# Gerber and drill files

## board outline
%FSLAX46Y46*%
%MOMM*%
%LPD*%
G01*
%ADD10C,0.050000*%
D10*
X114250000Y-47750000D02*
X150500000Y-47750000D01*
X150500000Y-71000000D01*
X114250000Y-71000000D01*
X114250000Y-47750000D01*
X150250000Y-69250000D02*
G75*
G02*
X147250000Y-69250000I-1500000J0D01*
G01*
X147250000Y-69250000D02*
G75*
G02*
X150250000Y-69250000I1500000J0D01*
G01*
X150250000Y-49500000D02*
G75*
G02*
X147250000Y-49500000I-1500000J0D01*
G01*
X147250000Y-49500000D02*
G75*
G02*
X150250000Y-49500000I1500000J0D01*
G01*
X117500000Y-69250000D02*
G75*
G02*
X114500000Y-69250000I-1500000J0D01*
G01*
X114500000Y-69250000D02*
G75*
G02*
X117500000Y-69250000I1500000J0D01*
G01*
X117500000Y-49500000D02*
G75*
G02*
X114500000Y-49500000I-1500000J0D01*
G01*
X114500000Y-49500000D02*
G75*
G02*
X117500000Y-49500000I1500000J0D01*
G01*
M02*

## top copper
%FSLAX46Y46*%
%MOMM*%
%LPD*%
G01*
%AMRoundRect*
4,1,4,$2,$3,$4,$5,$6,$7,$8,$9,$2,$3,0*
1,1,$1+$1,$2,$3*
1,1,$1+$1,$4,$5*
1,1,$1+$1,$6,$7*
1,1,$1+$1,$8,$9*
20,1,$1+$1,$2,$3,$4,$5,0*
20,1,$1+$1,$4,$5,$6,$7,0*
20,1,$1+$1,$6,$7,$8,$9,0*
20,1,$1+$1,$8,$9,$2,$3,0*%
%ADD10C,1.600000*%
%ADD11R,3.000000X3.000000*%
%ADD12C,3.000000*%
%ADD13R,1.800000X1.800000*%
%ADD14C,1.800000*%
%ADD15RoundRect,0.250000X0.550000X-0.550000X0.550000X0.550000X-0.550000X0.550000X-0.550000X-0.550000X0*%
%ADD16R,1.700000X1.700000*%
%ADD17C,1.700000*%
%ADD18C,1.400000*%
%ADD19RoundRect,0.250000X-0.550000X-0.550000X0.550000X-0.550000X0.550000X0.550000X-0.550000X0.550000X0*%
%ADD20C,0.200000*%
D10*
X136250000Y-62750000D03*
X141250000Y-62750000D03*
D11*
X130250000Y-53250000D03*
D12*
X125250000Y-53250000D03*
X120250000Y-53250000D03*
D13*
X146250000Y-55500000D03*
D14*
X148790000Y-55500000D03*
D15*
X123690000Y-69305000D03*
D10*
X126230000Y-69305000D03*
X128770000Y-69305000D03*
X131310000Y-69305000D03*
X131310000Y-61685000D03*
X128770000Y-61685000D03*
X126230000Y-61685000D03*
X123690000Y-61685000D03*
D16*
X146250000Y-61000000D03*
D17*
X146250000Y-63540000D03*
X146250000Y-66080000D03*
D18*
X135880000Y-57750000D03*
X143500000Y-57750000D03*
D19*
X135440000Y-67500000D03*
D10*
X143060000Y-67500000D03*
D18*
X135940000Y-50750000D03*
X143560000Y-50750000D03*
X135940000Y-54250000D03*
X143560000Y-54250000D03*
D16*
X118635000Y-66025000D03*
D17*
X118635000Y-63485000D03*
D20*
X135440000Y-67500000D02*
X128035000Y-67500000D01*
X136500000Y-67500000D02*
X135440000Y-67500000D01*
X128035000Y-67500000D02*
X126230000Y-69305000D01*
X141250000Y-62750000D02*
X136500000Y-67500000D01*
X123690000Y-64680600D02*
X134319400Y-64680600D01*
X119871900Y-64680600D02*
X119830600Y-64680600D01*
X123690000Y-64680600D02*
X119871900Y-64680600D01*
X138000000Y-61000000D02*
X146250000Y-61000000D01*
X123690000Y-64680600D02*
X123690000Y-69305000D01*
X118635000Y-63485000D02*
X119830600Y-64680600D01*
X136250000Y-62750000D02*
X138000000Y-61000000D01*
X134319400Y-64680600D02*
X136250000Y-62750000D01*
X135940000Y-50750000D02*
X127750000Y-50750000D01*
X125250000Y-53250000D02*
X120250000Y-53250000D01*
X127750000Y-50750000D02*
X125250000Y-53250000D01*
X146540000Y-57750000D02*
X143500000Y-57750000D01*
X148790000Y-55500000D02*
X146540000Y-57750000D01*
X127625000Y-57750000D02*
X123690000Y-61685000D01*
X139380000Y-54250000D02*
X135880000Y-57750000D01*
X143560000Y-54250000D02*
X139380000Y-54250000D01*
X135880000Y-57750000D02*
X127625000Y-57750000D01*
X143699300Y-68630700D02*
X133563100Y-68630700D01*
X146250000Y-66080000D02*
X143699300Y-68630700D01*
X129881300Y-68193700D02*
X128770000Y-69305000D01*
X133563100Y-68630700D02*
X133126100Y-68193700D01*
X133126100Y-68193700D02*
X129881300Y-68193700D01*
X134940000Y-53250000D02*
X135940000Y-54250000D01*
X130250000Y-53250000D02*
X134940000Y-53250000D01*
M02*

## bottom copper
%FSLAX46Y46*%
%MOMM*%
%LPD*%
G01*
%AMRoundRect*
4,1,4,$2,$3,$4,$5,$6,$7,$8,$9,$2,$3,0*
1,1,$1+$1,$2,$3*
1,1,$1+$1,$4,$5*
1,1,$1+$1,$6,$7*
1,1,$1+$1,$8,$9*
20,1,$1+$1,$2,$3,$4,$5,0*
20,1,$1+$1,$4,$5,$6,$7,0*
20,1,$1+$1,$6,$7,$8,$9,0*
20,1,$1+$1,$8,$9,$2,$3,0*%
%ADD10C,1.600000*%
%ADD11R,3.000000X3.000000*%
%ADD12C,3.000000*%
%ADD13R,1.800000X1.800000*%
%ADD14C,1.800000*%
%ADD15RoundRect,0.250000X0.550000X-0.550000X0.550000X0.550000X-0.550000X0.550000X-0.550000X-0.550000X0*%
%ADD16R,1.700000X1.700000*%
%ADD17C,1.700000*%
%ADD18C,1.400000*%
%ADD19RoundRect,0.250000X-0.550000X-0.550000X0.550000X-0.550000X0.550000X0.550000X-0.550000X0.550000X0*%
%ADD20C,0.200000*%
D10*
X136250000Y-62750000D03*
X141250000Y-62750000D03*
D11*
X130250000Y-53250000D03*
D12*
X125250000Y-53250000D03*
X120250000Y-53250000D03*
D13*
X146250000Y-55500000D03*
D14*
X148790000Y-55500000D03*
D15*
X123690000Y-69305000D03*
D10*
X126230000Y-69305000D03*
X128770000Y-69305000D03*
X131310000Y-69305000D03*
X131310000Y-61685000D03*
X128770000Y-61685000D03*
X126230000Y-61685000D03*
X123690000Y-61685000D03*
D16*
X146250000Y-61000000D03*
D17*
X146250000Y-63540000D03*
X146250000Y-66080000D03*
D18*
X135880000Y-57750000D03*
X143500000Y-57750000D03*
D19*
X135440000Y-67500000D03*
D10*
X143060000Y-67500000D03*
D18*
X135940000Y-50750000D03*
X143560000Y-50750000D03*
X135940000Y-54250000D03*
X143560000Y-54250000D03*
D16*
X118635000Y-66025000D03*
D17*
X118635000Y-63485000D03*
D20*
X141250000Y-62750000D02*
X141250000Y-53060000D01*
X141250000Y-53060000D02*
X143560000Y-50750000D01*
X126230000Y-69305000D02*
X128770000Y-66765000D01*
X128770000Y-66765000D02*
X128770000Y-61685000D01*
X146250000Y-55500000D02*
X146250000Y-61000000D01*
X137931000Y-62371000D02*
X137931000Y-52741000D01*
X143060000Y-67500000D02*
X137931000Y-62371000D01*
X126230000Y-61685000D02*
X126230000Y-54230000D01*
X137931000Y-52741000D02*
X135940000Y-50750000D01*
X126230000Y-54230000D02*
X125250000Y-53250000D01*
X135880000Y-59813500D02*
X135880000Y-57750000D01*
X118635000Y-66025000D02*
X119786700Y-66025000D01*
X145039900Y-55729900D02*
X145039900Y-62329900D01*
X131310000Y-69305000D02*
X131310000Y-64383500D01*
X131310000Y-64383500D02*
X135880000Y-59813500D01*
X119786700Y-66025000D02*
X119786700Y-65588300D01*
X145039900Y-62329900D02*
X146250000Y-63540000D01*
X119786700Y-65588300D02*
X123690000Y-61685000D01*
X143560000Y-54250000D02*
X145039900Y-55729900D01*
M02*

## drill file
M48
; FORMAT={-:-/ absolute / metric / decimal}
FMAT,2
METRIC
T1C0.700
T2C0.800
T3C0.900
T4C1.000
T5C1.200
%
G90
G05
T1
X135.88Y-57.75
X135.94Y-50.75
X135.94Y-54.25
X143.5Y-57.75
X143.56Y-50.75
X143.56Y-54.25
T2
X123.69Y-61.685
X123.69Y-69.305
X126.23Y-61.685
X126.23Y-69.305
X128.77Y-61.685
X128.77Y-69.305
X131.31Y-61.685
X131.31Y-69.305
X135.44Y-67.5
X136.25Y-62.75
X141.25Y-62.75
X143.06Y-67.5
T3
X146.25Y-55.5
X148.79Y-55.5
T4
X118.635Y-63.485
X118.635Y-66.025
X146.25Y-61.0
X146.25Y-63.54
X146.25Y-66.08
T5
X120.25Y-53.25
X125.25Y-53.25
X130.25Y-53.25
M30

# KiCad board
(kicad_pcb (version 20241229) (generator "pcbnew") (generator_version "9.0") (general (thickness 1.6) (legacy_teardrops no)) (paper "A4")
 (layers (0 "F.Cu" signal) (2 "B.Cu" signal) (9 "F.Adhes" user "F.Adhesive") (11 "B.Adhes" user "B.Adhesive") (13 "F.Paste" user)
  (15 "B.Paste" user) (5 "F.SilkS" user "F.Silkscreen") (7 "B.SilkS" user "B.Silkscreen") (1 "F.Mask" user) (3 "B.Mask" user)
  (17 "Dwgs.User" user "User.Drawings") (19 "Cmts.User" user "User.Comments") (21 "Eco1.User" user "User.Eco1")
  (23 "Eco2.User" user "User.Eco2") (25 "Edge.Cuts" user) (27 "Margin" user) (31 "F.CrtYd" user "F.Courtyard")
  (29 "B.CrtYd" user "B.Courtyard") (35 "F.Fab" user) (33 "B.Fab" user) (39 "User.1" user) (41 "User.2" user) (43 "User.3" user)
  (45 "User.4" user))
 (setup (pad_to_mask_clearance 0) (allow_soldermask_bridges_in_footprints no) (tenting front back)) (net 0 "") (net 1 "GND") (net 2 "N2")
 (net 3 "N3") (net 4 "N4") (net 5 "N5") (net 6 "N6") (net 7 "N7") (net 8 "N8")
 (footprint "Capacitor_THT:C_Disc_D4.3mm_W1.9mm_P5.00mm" (layer "F.Cu") (at 136.25 62.75)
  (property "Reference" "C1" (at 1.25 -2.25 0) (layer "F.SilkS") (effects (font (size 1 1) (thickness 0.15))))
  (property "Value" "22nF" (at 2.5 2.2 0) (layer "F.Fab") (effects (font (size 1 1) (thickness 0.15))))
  (pad "1" thru_hole circle (at 0 0) (size 1.6 1.6) (drill 0.8) (layers "*.Cu" "*.Mask") (remove_unused_layers no) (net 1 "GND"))
  (pad "2" thru_hole circle (at 5 0) (size 1.6 1.6) (drill 0.8) (layers "*.Cu" "*.Mask") (remove_unused_layers no) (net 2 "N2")))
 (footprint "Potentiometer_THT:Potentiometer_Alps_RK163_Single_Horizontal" (layer "F.Cu") (at 130.25 53.25 -90)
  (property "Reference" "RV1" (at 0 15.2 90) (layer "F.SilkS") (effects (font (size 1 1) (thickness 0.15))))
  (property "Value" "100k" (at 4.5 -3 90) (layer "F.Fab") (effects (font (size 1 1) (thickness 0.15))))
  (pad "1" thru_hole rect (at 0 0 90) (size 3 3) (drill 1.2) (layers "*.Cu" "*.Mask") (remove_unused_layers no) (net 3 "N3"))
  (pad "2" thru_hole circle (at 0 5 90) (size 3 3) (drill 1.2) (layers "*.Cu" "*.Mask") (remove_unused_layers no) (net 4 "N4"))
  (pad "3" thru_hole circle (at 0 10 90) (size 3 3) (drill 1.2) (layers "*.Cu" "*.Mask") (remove_unused_layers no) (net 4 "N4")))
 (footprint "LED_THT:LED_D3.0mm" (layer "F.Cu") (at 146.25 55.5)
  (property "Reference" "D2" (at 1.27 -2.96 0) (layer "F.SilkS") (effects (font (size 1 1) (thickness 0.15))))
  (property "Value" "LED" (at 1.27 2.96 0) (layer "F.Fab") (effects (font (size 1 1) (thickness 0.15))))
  (pad "1" thru_hole rect (at 0 0) (size 1.8 1.8) (drill 0.9) (layers "*.Cu" "*.Mask") (remove_unused_layers no) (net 1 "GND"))
  (pad "2" thru_hole circle (at 2.54 0) (size 1.8 1.8) (drill 0.9) (layers "*.Cu" "*.Mask") (remove_unused_layers no) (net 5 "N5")))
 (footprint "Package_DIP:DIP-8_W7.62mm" (layer "F.Cu") (at 123.69 69.305 90)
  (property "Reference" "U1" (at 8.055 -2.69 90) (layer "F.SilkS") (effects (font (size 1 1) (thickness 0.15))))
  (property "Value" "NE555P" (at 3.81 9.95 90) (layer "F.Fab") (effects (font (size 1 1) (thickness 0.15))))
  (pad "1" thru_hole roundrect (at 0 0 90) (size 1.6 1.6) (drill 0.8) (layers "*.Cu" "*.Mask") (remove_unused_layers no)
   (roundrect_rratio 0.15625) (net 1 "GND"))
  (pad "2" thru_hole circle (at 0 2.54 90) (size 1.6 1.6) (drill 0.8) (layers "*.Cu" "*.Mask") (remove_unused_layers no) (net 2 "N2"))
  (pad "3" thru_hole circle (at 0 5.08 90) (size 1.6 1.6) (drill 0.8) (layers "*.Cu" "*.Mask") (remove_unused_layers no) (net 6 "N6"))
  (pad "4" thru_hole circle (at 0 7.62 90) (size 1.6 1.6) (drill 0.8) (layers "*.Cu" "*.Mask") (remove_unused_layers no) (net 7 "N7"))
  (pad "5" thru_hole circle (at 7.62 7.62 90) (size 1.6 1.6) (drill 0.8) (layers "*.Cu" "*.Mask") (remove_unused_layers no) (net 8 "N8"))
  (pad "6" thru_hole circle (at 7.62 5.08 90) (size 1.6 1.6) (drill 0.8) (layers "*.Cu" "*.Mask") (remove_unused_layers no) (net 2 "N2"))
  (pad "7" thru_hole circle (at 7.62 2.54 90) (size 1.6 1.6) (drill 0.8) (layers "*.Cu" "*.Mask") (remove_unused_layers no) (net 4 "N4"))
  (pad "8" thru_hole circle (at 7.62 0 90) (size 1.6 1.6) (drill 0.8) (layers "*.Cu" "*.Mask") (remove_unused_layers no) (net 7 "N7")))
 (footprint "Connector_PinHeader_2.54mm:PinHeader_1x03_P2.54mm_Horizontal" (layer "F.Cu") (at 146.25 61)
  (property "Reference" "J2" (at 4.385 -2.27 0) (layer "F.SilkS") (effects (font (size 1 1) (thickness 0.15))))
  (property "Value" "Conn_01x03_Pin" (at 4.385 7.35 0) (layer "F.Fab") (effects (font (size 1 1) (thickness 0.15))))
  (pad "1" thru_hole rect (at 0 0) (size 1.7 1.7) (drill 1) (layers "*.Cu" "*.Mask") (remove_unused_layers no) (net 1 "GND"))
  (pad "2" thru_hole circle (at 0 2.54) (size 1.7 1.7) (drill 1) (layers "*.Cu" "*.Mask") (remove_unused_layers no) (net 7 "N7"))
  (pad "3" thru_hole circle (at 0 5.08) (size 1.7 1.7) (drill 1) (layers "*.Cu" "*.Mask") (remove_unused_layers no) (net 6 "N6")))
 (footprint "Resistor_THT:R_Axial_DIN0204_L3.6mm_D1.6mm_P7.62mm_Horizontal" (layer "F.Cu") (at 135.88 57.75)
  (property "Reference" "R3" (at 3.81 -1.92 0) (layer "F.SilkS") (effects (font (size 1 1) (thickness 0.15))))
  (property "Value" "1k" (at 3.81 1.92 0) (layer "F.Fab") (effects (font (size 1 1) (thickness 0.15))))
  (pad "1" thru_hole circle (at 0 0) (size 1.4 1.4) (drill 0.7) (layers "*.Cu" "*.Mask") (remove_unused_layers no) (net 7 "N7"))
  (pad "2" thru_hole circle (at 7.62 0) (size 1.4 1.4) (drill 0.7) (layers "*.Cu" "*.Mask") (remove_unused_layers no) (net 5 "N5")))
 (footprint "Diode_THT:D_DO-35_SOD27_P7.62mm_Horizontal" (layer "F.Cu") (at 135.44 67.5)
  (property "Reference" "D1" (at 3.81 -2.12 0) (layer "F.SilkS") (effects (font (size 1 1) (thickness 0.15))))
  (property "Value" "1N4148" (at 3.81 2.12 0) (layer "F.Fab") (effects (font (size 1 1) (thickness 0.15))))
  (pad "1" thru_hole roundrect (at 0 0) (size 1.6 1.6) (drill 0.8) (layers "*.Cu" "*.Mask") (remove_unused_layers no)
   (roundrect_rratio 0.15625) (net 2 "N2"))
  (pad "2" thru_hole circle (at 7.62 0) (size 1.6 1.6) (drill 0.8) (layers "*.Cu" "*.Mask") (remove_unused_layers no) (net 4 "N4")))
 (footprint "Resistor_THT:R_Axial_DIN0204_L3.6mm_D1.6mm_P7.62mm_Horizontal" (layer "F.Cu") (at 135.94 50.75)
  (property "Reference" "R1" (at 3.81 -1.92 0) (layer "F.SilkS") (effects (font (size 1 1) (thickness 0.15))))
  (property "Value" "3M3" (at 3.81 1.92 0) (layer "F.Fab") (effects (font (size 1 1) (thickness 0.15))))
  (pad "1" thru_hole circle (at 0 0) (size 1.4 1.4) (drill 0.7) (layers "*.Cu" "*.Mask") (remove_unused_layers no) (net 4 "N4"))
  (pad "2" thru_hole circle (at 7.62 0) (size 1.4 1.4) (drill 0.7) (layers "*.Cu" "*.Mask") (remove_unused_layers no) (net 2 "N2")))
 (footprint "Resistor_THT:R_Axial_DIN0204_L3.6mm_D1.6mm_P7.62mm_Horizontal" (layer "F.Cu") (at 135.94 54.25)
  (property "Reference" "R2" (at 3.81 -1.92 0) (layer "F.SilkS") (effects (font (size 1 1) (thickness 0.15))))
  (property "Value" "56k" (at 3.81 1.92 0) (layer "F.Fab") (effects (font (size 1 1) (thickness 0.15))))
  (pad "1" thru_hole circle (at 0 0) (size 1.4 1.4) (drill 0.7) (layers "*.Cu" "*.Mask") (remove_unused_layers no) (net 3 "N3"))
  (pad "2" thru_hole circle (at 7.62 0) (size 1.4 1.4) (drill 0.7) (layers "*.Cu" "*.Mask") (remove_unused_layers no) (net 7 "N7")))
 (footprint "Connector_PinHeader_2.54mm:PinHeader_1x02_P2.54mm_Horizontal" (layer "F.Cu") (at 118.635 66.025 180)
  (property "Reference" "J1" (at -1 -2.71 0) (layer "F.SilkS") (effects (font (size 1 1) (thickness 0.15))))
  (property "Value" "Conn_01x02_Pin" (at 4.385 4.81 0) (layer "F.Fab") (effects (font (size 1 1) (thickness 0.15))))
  (pad "1" thru_hole rect (at 0 0 180) (size 1.7 1.7) (drill 1) (layers "*.Cu" "*.Mask") (remove_unused_layers no) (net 7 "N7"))
  (pad "2" thru_hole circle (at 0 2.54 180) (size 1.7 1.7) (drill 1) (layers "*.Cu" "*.Mask") (remove_unused_layers no) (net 1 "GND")))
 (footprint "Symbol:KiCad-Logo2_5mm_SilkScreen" (layer "B.Cu") (at 124.5 57.75 180)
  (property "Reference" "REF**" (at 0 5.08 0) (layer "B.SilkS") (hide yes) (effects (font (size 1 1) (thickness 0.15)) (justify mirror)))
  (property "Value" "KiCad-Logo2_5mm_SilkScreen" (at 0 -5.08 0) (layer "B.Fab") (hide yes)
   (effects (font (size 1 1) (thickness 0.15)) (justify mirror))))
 (gr_rect (start 114.25 47.75) (end 150.5 71) (stroke (width 0.05) (type default)) (fill no) (layer "Edge.Cuts"))
 (gr_circle (center 148.75 69.25) (end 150.25 69.25) (stroke (width 0.05) (type solid)) (fill no) (layer "Edge.Cuts"))
 (gr_circle (center 148.75 49.5) (end 150.25 49.5) (stroke (width 0.05) (type solid)) (fill no) (layer "Edge.Cuts"))
 (gr_circle (center 116 69.25) (end 117.5 69.25) (stroke (width 0.05) (type solid)) (fill no) (layer "Edge.Cuts"))
 (gr_circle (center 116 49.5) (end 117.5 49.5) (stroke (width 0.05) (type solid)) (fill no) (layer "Edge.Cuts"))
 (segment (start 135.44 67.5) (end 128.035 67.5) (width 0.2) (layer "F.Cu") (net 2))
 (segment (start 136.5 67.5) (end 135.44 67.5) (width 0.2) (layer "F.Cu") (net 2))
 (segment (start 128.035 67.5) (end 126.23 69.305) (width 0.2) (layer "F.Cu") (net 2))
 (segment (start 141.25 62.75) (end 136.5 67.5) (width 0.2) (layer "F.Cu") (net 2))
 (segment (start 141.25 62.75) (end 141.25 53.06) (width 0.2) (layer "B.Cu") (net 2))
 (segment (start 141.25 53.06) (end 143.56 50.75) (width 0.2) (layer "B.Cu") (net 2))
 (segment (start 126.23 69.305) (end 128.77 66.765) (width 0.2) (layer "B.Cu") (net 2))
 (segment (start 128.77 66.765) (end 128.77 61.685) (width 0.2) (layer "B.Cu") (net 2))
 (segment (start 123.69 64.6806) (end 134.3194 64.6806) (width 0.2) (layer "F.Cu") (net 1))
 (segment (start 119.8719 64.6806) (end 119.8306 64.6806) (width 0.2) (layer "F.Cu") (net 1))
 (segment (start 123.69 64.6806) (end 119.8719 64.6806) (width 0.2) (layer "F.Cu") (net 1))
 (segment (start 138 61) (end 146.25 61) (width 0.2) (layer "F.Cu") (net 1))
 (segment (start 123.69 64.6806) (end 123.69 69.305) (width 0.2) (layer "F.Cu") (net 1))
 (segment (start 118.635 63.485) (end 119.8306 64.6806) (width 0.2) (layer "F.Cu") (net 1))
 (segment (start 136.25 62.75) (end 138 61) (width 0.2) (layer "F.Cu") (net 1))
 (segment (start 134.3194 64.6806) (end 136.25 62.75) (width 0.2) (layer "F.Cu") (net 1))
 (segment (start 146.25 55.5) (end 146.25 61) (width 0.2) (layer "B.Cu") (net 1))
 (segment (start 135.94 50.75) (end 127.75 50.75) (width 0.2) (layer "F.Cu") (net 4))
 (segment (start 125.25 53.25) (end 120.25 53.25) (width 0.2) (layer "F.Cu") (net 4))
 (segment (start 127.75 50.75) (end 125.25 53.25) (width 0.2) (layer "F.Cu") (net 4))
 (segment (start 137.931 62.371) (end 137.931 52.741) (width 0.2) (layer "B.Cu") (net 4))
 (segment (start 143.06 67.5) (end 137.931 62.371) (width 0.2) (layer "B.Cu") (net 4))
 (segment (start 126.23 61.685) (end 126.23 54.23) (width 0.2) (layer "B.Cu") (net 4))
 (segment (start 137.931 52.741) (end 135.94 50.75) (width 0.2) (layer "B.Cu") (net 4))
 (segment (start 126.23 54.23) (end 125.25 53.25) (width 0.2) (layer "B.Cu") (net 4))
 (segment (start 146.54 57.75) (end 143.5 57.75) (width 0.2) (layer "F.Cu") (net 5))
 (segment (start 148.79 55.5) (end 146.54 57.75) (width 0.2) (layer "F.Cu") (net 5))
 (segment (start 127.625 57.75) (end 123.69 61.685) (width 0.2) (layer "F.Cu") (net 7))
 (segment (start 139.38 54.25) (end 135.88 57.75) (width 0.2) (layer "F.Cu") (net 7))
 (segment (start 143.56 54.25) (end 139.38 54.25) (width 0.2) (layer "F.Cu") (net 7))
 (segment (start 135.88 57.75) (end 127.625 57.75) (width 0.2) (layer "F.Cu") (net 7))
 (segment (start 135.88 59.8135) (end 135.88 57.75) (width 0.2) (layer "B.Cu") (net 7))
 (segment (start 118.635 66.025) (end 119.7867 66.025) (width 0.2) (layer "B.Cu") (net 7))
 (segment (start 145.0399 55.7299) (end 145.0399 62.3299) (width 0.2) (layer "B.Cu") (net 7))
 (segment (start 131.31 69.305) (end 131.31 64.3835) (width 0.2) (layer "B.Cu") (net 7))
 (segment (start 131.31 64.3835) (end 135.88 59.8135) (width 0.2) (layer "B.Cu") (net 7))
 (segment (start 119.7867 66.025) (end 119.7867 65.5883) (width 0.2) (layer "B.Cu") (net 7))
 (segment (start 145.0399 62.3299) (end 146.25 63.54) (width 0.2) (layer "B.Cu") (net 7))
 (segment (start 119.7867 65.5883) (end 123.69 61.685) (width 0.2) (layer "B.Cu") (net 7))
 (segment (start 143.56 54.25) (end 145.0399 55.7299) (width 0.2) (layer "B.Cu") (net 7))
 (segment (start 143.6993 68.6307) (end 133.5631 68.6307) (width 0.2) (layer "F.Cu") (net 6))
 (segment (start 146.25 66.08) (end 143.6993 68.6307) (width 0.2) (layer "F.Cu") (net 6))
 (segment (start 129.8813 68.1937) (end 128.77 69.305) (width 0.2) (layer "F.Cu") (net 6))
 (segment (start 133.5631 68.6307) (end 133.1261 68.1937) (width 0.2) (layer "F.Cu") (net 6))
 (segment (start 133.1261 68.1937) (end 129.8813 68.1937) (width 0.2) (layer "F.Cu") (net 6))
 (segment (start 134.94 53.25) (end 135.94 54.25) (width 0.2) (layer "F.Cu") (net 3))
 (segment (start 130.25 53.25) (end 134.94 53.25) (width 0.2) (layer "F.Cu") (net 3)))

